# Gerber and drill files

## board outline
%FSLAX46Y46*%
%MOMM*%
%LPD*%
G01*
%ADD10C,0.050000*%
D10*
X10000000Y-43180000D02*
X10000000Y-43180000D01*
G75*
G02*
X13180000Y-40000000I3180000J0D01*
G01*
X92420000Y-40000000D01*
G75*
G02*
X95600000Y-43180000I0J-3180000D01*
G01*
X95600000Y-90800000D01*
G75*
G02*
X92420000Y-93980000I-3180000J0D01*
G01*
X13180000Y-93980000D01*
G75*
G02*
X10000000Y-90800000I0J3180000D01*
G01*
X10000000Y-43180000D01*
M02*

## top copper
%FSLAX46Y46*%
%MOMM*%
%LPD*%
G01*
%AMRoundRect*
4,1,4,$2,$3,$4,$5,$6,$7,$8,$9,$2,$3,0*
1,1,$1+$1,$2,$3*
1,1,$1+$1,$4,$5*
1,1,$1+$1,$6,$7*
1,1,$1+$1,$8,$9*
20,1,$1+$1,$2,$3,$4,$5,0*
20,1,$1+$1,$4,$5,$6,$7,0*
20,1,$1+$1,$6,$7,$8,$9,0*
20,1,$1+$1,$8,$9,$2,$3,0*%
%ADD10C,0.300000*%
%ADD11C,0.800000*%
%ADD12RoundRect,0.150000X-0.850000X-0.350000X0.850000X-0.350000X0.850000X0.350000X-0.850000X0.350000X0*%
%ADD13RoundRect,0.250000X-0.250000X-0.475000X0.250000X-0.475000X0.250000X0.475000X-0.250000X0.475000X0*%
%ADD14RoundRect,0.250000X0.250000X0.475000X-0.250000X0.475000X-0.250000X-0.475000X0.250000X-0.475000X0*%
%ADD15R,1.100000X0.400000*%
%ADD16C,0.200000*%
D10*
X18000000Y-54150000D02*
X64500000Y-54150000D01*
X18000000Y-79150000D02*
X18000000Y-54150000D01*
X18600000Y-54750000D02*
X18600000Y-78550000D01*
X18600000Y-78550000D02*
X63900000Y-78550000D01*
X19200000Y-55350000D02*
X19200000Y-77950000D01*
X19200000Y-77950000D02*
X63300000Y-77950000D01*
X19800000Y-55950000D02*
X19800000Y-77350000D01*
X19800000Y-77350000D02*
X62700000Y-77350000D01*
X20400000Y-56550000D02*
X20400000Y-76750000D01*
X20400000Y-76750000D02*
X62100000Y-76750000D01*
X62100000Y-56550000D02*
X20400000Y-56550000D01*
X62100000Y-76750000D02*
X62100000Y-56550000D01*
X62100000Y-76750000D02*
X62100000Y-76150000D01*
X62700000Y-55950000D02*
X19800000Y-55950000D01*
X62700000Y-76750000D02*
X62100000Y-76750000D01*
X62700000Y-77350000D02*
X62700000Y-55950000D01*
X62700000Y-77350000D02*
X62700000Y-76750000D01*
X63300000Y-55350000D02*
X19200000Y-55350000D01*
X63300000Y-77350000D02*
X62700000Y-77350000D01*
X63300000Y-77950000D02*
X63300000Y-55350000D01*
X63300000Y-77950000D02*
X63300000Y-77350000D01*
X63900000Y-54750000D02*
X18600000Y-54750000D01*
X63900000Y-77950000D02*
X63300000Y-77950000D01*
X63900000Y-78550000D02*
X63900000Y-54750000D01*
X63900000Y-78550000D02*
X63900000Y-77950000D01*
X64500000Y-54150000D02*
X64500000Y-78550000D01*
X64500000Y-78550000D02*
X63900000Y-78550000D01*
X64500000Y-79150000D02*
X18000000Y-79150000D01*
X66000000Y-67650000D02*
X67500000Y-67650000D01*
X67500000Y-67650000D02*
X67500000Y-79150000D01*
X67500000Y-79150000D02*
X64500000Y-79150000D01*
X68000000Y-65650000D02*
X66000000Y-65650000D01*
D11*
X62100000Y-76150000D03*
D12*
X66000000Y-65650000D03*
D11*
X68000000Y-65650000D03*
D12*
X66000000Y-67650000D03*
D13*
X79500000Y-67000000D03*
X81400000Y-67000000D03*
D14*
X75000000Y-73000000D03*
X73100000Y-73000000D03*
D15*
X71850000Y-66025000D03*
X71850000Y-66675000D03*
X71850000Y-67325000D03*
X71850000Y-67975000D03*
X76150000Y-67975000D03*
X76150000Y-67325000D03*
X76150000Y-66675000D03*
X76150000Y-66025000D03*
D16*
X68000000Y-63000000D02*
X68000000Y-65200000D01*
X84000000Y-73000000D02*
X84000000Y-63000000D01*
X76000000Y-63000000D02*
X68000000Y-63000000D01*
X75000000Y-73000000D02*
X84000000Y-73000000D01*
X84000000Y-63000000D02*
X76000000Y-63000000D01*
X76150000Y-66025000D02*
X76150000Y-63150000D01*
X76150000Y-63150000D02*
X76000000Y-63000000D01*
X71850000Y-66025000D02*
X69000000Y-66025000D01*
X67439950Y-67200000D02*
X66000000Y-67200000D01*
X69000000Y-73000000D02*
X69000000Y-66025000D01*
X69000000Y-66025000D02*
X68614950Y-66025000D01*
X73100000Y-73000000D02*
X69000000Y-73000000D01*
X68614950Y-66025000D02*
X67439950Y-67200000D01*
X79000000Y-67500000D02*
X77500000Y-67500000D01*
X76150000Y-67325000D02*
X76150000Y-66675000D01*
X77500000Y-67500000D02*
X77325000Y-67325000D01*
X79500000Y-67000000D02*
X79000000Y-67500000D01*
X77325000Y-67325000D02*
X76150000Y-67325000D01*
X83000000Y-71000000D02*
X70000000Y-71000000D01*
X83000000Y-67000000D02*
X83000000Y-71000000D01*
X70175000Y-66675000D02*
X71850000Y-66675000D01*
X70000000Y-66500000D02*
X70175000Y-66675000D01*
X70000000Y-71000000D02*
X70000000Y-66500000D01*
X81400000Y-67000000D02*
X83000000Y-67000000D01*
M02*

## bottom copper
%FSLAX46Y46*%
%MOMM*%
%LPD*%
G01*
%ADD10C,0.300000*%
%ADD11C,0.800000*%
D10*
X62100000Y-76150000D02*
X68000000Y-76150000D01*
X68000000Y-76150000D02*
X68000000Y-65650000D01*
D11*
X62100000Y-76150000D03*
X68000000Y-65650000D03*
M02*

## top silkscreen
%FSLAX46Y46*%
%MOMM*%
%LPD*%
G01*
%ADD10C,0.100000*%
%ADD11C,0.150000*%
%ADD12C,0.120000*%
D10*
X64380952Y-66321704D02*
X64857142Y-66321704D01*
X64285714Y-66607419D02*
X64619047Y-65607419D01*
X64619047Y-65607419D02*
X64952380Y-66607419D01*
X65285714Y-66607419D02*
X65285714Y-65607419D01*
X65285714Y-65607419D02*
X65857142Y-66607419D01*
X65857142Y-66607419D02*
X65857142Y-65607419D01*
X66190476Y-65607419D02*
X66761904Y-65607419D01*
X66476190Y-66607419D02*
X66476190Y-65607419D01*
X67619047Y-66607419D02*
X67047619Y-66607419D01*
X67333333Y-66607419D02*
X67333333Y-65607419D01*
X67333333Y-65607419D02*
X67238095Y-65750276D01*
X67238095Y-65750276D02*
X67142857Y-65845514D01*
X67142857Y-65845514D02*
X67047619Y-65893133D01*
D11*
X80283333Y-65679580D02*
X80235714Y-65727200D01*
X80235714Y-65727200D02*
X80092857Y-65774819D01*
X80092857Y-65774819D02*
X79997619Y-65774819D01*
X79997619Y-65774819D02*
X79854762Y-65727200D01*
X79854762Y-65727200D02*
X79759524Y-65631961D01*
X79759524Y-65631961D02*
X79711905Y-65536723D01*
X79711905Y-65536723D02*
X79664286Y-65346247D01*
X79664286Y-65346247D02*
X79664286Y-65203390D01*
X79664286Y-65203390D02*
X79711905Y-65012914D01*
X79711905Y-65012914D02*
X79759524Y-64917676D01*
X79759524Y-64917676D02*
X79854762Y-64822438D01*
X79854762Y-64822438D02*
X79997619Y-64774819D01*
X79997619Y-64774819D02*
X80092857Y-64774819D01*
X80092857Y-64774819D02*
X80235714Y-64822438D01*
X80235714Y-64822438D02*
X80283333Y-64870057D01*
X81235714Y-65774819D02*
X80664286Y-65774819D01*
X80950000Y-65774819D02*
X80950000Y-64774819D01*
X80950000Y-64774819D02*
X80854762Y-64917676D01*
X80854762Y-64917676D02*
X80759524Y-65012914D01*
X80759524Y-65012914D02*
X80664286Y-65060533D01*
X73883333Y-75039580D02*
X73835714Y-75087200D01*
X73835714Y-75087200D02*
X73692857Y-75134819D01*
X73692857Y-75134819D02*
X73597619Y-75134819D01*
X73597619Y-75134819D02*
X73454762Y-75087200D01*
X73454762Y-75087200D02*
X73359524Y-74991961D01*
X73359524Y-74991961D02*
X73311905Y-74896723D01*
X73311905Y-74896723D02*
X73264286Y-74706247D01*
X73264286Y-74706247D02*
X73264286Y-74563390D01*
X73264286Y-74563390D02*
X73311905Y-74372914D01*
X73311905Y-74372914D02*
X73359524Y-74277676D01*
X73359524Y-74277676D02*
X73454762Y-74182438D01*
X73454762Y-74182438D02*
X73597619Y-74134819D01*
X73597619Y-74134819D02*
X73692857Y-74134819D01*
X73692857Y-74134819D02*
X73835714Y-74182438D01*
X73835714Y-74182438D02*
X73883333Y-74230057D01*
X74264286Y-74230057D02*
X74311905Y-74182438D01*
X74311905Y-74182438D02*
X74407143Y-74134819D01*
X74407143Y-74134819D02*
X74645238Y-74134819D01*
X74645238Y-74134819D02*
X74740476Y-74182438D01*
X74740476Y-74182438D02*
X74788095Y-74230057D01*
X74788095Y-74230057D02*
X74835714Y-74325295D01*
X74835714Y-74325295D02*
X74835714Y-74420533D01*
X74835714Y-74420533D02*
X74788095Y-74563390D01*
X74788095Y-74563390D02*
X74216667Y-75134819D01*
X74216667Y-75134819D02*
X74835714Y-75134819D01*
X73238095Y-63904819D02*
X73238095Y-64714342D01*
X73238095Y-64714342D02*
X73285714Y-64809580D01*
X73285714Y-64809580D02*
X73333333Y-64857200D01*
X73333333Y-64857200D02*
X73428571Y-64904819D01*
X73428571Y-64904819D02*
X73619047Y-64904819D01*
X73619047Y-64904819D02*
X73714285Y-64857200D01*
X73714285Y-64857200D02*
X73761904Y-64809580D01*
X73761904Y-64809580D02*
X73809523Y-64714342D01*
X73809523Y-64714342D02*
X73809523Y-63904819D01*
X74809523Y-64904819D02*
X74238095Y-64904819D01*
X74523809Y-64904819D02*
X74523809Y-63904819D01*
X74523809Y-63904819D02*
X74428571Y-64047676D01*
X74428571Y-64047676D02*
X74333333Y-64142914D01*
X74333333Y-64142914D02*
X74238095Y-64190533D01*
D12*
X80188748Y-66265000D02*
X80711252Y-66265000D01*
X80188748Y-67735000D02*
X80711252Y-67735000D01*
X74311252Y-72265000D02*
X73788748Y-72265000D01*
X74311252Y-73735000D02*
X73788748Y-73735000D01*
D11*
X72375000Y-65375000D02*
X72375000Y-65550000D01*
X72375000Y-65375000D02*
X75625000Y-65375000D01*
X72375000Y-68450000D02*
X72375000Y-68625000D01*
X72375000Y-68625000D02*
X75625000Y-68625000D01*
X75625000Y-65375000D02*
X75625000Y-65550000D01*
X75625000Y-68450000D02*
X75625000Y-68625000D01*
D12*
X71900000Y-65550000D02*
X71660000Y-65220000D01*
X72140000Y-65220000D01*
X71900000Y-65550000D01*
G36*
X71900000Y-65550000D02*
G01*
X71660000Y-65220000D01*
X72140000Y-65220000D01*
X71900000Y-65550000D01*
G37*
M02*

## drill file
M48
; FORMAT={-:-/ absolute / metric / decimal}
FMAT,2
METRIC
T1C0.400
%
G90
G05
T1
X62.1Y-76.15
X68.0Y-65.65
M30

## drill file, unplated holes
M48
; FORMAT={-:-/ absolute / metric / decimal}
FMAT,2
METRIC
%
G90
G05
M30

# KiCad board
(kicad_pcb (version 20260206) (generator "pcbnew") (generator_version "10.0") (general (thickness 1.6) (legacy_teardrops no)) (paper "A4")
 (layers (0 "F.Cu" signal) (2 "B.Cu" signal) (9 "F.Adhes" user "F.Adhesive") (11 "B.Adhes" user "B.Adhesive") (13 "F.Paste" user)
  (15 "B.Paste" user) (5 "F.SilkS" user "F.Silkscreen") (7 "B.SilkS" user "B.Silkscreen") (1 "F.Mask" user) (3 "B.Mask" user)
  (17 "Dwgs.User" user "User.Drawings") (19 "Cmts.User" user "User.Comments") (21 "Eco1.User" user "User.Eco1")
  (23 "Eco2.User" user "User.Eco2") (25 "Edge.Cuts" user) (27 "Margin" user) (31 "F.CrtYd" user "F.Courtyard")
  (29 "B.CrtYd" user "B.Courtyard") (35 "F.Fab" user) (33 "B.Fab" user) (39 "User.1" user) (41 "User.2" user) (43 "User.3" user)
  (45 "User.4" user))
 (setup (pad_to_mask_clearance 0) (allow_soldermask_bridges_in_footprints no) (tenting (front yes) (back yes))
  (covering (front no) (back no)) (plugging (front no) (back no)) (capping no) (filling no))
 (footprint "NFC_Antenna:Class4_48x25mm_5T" (layer "F.Cu") (at 66 66.65)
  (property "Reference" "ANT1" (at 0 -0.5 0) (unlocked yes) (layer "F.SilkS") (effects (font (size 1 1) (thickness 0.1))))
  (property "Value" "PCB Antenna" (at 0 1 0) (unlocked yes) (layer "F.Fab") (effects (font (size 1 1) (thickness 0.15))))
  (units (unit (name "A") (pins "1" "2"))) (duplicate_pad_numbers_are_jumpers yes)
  (fp_line (start -48 -12.5) (end -1.5 -12.5) (stroke (width 0.3) (type solid)) (layer "F.Cu"))
  (fp_line (start -48 12.5) (end -48 -12.5) (stroke (width 0.3) (type solid)) (layer "F.Cu"))
  (fp_line (start -47.4 -11.9) (end -47.4 11.9) (stroke (width 0.3) (type solid)) (layer "F.Cu"))
  (fp_line (start -47.4 11.9) (end -2.1 11.9) (stroke (width 0.3) (type solid)) (layer "F.Cu"))
  (fp_line (start -46.8 -11.3) (end -46.8 11.3) (stroke (width 0.3) (type solid)) (layer "F.Cu"))
  (fp_line (start -46.8 11.3) (end -2.7 11.3) (stroke (width 0.3) (type solid)) (layer "F.Cu"))
  (fp_line (start -46.2 -10.7) (end -46.2 10.7) (stroke (width 0.3) (type solid)) (layer "F.Cu"))
  (fp_line (start -46.2 10.7) (end -3.3 10.7) (stroke (width 0.3) (type solid)) (layer "F.Cu"))
  (fp_line (start -45.6 -10.1) (end -45.6 10.1) (stroke (width 0.3) (type solid)) (layer "F.Cu"))
  (fp_line (start -45.6 10.1) (end -3.9 10.1) (stroke (width 0.3) (type solid)) (layer "F.Cu"))
  (fp_line (start -3.9 -10.1) (end -45.6 -10.1) (stroke (width 0.3) (type solid)) (layer "F.Cu"))
  (fp_line (start -3.9 10.1) (end -3.9 -10.1) (stroke (width 0.3) (type solid)) (layer "F.Cu"))
  (fp_line (start -3.9 10.1) (end -3.9 9.5) (stroke (width 0.3) (type solid)) (layer "F.Cu"))
  (fp_line (start -3.3 -10.7) (end -46.2 -10.7) (stroke (width 0.3) (type solid)) (layer "F.Cu"))
  (fp_line (start -3.3 10.1) (end -3.9 10.1) (stroke (width 0.3) (type solid)) (layer "F.Cu"))
  (fp_line (start -3.3 10.7) (end -3.3 -10.7) (stroke (width 0.3) (type solid)) (layer "F.Cu"))
  (fp_line (start -3.3 10.7) (end -3.3 10.1) (stroke (width 0.3) (type solid)) (layer "F.Cu"))
  (fp_line (start -2.7 -11.3) (end -46.8 -11.3) (stroke (width 0.3) (type solid)) (layer "F.Cu"))
  (fp_line (start -2.7 10.7) (end -3.3 10.7) (stroke (width 0.3) (type solid)) (layer "F.Cu"))
  (fp_line (start -2.7 11.3) (end -2.7 -11.3) (stroke (width 0.3) (type solid)) (layer "F.Cu"))
  (fp_line (start -2.7 11.3) (end -2.7 10.7) (stroke (width 0.3) (type solid)) (layer "F.Cu"))
  (fp_line (start -2.1 -11.9) (end -47.4 -11.9) (stroke (width 0.3) (type solid)) (layer "F.Cu"))
  (fp_line (start -2.1 11.3) (end -2.7 11.3) (stroke (width 0.3) (type solid)) (layer "F.Cu"))
  (fp_line (start -2.1 11.9) (end -2.1 -11.9) (stroke (width 0.3) (type solid)) (layer "F.Cu"))
  (fp_line (start -2.1 11.9) (end -2.1 11.3) (stroke (width 0.3) (type solid)) (layer "F.Cu"))
  (fp_line (start -1.5 -12.5) (end -1.5 11.9) (stroke (width 0.3) (type solid)) (layer "F.Cu"))
  (fp_line (start -1.5 11.9) (end -2.1 11.9) (stroke (width 0.3) (type solid)) (layer "F.Cu"))
  (fp_line (start -1.5 12.5) (end -48 12.5) (stroke (width 0.3) (type solid)) (layer "F.Cu"))
  (fp_line (start 0 1) (end 1.5 1) (stroke (width 0.3) (type solid)) (layer "F.Cu"))
  (fp_line (start 1.5 1) (end 1.5 12.5) (stroke (width 0.3) (type solid)) (layer "F.Cu"))
  (fp_line (start 1.5 12.5) (end -1.5 12.5) (stroke (width 0.3) (type solid)) (layer "F.Cu"))
  (fp_line (start 2 -1) (end 0 -1) (stroke (width 0.3) (type solid)) (layer "F.Cu"))
  (fp_line (start -3.9 9.5) (end 2 9.5) (stroke (width 0.3) (type solid)) (layer "B.Cu"))
  (fp_line (start 2 9.5) (end 2 -1) (stroke (width 0.3) (type solid)) (layer "B.Cu"))
  (pad "1" thru_hole circle (at -3.9 9.5) (size 0.8 0.8) (drill 0.4) (layers "*.Cu" "*.Mask") (remove_unused_layers no) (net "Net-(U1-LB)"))
  (pad "1" smd roundrect (at 0 -1) (size 2 1) (layers "F.Cu" "F.Mask") (roundrect_rratio 0.15) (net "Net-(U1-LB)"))
  (pad "1" thru_hole circle (at 2 -1) (size 0.8 0.8) (drill 0.4) (layers "*.Cu" "*.Mask") (remove_unused_layers no) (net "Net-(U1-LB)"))
  (pad "2" smd roundrect (at 0 1) (size 2 1) (layers "F.Cu" "F.Mask") (roundrect_rratio 0.15) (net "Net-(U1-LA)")))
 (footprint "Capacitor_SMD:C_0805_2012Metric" (layer "F.Cu") (at 80.45 67)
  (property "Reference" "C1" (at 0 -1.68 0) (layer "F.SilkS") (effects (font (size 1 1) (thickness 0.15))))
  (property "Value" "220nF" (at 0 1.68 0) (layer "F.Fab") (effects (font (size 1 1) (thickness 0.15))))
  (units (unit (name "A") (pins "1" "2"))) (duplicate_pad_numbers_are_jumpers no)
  (fp_line (start -0.261252 -0.735) (end 0.261252 -0.735) (stroke (width 0.12) (type solid)) (layer "F.SilkS"))
  (fp_line (start -0.261252 0.735) (end 0.261252 0.735) (stroke (width 0.12) (type solid)) (layer "F.SilkS"))
  (pad "1" smd roundrect (at -0.95 0) (size 1 1.45) (layers "F.Cu" "F.Mask" "F.Paste") (roundrect_rratio 0.25) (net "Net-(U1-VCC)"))
  (pad "2" smd roundrect (at 0.95 0) (size 1 1.45) (layers "F.Cu" "F.Mask" "F.Paste") (roundrect_rratio 0.25) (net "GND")))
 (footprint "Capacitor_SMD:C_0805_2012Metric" (layer "F.Cu") (at 74.05 73 180)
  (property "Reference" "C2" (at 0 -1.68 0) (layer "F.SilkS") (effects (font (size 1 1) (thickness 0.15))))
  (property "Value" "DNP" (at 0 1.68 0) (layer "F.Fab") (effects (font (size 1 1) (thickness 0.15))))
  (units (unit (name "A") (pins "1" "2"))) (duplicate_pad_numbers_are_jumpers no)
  (fp_line (start -0.261252 0.735) (end 0.261252 0.735) (stroke (width 0.12) (type solid)) (layer "F.SilkS"))
  (fp_line (start -0.261252 -0.735) (end 0.261252 -0.735) (stroke (width 0.12) (type solid)) (layer "F.SilkS"))
  (pad "1" smd roundrect (at -0.95 0 180) (size 1 1.45) (layers "F.Cu" "F.Mask" "F.Paste") (roundrect_rratio 0.25) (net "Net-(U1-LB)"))
  (pad "2" smd roundrect (at 0.95 0 180) (size 1 1.45) (layers "F.Cu" "F.Mask" "F.Paste") (roundrect_rratio 0.25) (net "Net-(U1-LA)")))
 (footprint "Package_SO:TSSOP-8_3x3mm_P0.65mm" (layer "F.Cu") (at 74 67)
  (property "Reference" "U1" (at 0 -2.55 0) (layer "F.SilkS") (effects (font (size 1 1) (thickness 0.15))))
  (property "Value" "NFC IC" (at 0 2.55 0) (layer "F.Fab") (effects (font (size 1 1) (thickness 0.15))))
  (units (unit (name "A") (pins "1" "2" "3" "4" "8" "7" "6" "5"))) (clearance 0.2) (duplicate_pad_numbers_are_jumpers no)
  (fp_line (start -1.625 -1.625) (end -1.625 -1.45) (stroke (width 0.15) (type solid)) (layer "F.SilkS"))
  (fp_line (start -1.625 -1.625) (end 1.625 -1.625) (stroke (width 0.15) (type solid)) (layer "F.SilkS"))
  (fp_line (start -1.625 1.45) (end -1.625 1.625) (stroke (width 0.15) (type solid)) (layer "F.SilkS"))
  (fp_line (start -1.625 1.625) (end 1.625 1.625) (stroke (width 0.15) (type solid)) (layer "F.SilkS"))
  (fp_line (start 1.625 -1.625) (end 1.625 -1.45) (stroke (width 0.15) (type solid)) (layer "F.SilkS"))
  (fp_line (start 1.625 1.45) (end 1.625 1.625) (stroke (width 0.15) (type solid)) (layer "F.SilkS"))
  (fp_poly
   (pts (xy -2.1 -1.45) (xy -2.34 -1.78) (xy -1.86 -1.78) (xy -2.1 -1.45)) (stroke (width 0.12) (type solid)) (fill yes) (layer "F.SilkS"))
  (pad "1" smd rect (at -2.15 -0.975) (size 1.1 0.4) (layers "F.Cu" "F.Mask" "F.Paste") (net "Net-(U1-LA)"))
  (pad "2" smd rect (at -2.15 -0.325) (size 1.1 0.4) (layers "F.Cu" "F.Mask" "F.Paste") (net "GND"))
  (pad "3" smd rect (at -2.15 0.325) (size 1.1 0.4) (layers "F.Cu" "F.Mask" "F.Paste") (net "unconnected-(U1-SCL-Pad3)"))
  (pad "4" smd rect (at -2.15 0.975) (size 1.1 0.4) (layers "F.Cu" "F.Mask" "F.Paste") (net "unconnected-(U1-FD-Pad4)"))
  (pad "5" smd rect (at 2.15 0.975) (size 1.1 0.4) (layers "F.Cu" "F.Mask" "F.Paste") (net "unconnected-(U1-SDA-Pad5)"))
  (pad "6" smd rect (at 2.15 0.325) (size 1.1 0.4) (layers "F.Cu" "F.Mask" "F.Paste") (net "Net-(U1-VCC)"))
  (pad "7" smd rect (at 2.15 -0.325) (size 1.1 0.4) (layers "F.Cu" "F.Mask" "F.Paste") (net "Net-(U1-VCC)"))
  (pad "8" smd rect (at 2.15 -0.975) (size 1.1 0.4) (layers "F.Cu" "F.Mask" "F.Paste") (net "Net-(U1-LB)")))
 (gr_rect (start 10 40) (end 95.6 93.98) (radius 3.18) (stroke (width 0.05) (type solid)) (fill no) (layer "Edge.Cuts"))
 (segment (start 68 63) (end 68 65.2) (width 0.2) (layer "F.Cu") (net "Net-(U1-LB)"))
 (segment (start 84 73) (end 84 63) (width 0.2) (layer "F.Cu") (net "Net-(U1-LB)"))
 (segment (start 76 63) (end 68 63) (width 0.2) (layer "F.Cu") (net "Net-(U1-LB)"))
 (segment (start 75 73) (end 84 73) (width 0.2) (layer "F.Cu") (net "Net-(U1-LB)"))
 (segment (start 84 63) (end 76 63) (width 0.2) (layer "F.Cu") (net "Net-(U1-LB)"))
 (segment (start 76.15 66.025) (end 76.15 63.15) (width 0.2) (layer "F.Cu") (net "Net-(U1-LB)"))
 (segment (start 76.15 63.15) (end 76 63) (width 0.2) (layer "F.Cu") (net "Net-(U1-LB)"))
 (segment (start 71.85 66.025) (end 69 66.025) (width 0.2) (layer "F.Cu") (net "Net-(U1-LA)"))
 (segment (start 67.43995 67.2) (end 66 67.2) (width 0.2) (layer "F.Cu") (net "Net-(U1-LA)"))
 (segment (start 69 73) (end 69 66.025) (width 0.2) (layer "F.Cu") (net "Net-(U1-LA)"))
 (segment (start 69 66.025) (end 68.61495 66.025) (width 0.2) (layer "F.Cu") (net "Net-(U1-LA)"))
 (segment (start 73.1 73) (end 69 73) (width 0.2) (layer "F.Cu") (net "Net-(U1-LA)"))
 (segment (start 68.61495 66.025) (end 67.43995 67.2) (width 0.2) (layer "F.Cu") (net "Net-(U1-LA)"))
 (segment (start 79 67.5) (end 77.5 67.5) (width 0.2) (layer "F.Cu") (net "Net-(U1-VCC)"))
 (segment (start 76.15 67.325) (end 76.15 66.675) (width 0.2) (layer "F.Cu") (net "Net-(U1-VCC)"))
 (segment (start 77.5 67.5) (end 77.325 67.325) (width 0.2) (layer "F.Cu") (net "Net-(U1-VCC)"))
 (segment (start 79.5 67) (end 79 67.5) (width 0.2) (layer "F.Cu") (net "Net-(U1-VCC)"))
 (segment (start 77.325 67.325) (end 76.15 67.325) (width 0.2) (layer "F.Cu") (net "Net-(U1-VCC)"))
 (segment (start 83 71) (end 70 71) (width 0.2) (layer "F.Cu") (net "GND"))
 (segment (start 83 67) (end 83 71) (width 0.2) (layer "F.Cu") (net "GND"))
 (segment (start 70.175 66.675) (end 71.85 66.675) (width 0.2) (layer "F.Cu") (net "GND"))
 (segment (start 70 66.5) (end 70.175 66.675) (width 0.2) (layer "F.Cu") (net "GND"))
 (segment (start 70 71) (end 70 66.5) (width 0.2) (layer "F.Cu") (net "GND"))
 (segment (start 81.4 67) (end 83 67) (width 0.2) (layer "F.Cu") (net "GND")))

